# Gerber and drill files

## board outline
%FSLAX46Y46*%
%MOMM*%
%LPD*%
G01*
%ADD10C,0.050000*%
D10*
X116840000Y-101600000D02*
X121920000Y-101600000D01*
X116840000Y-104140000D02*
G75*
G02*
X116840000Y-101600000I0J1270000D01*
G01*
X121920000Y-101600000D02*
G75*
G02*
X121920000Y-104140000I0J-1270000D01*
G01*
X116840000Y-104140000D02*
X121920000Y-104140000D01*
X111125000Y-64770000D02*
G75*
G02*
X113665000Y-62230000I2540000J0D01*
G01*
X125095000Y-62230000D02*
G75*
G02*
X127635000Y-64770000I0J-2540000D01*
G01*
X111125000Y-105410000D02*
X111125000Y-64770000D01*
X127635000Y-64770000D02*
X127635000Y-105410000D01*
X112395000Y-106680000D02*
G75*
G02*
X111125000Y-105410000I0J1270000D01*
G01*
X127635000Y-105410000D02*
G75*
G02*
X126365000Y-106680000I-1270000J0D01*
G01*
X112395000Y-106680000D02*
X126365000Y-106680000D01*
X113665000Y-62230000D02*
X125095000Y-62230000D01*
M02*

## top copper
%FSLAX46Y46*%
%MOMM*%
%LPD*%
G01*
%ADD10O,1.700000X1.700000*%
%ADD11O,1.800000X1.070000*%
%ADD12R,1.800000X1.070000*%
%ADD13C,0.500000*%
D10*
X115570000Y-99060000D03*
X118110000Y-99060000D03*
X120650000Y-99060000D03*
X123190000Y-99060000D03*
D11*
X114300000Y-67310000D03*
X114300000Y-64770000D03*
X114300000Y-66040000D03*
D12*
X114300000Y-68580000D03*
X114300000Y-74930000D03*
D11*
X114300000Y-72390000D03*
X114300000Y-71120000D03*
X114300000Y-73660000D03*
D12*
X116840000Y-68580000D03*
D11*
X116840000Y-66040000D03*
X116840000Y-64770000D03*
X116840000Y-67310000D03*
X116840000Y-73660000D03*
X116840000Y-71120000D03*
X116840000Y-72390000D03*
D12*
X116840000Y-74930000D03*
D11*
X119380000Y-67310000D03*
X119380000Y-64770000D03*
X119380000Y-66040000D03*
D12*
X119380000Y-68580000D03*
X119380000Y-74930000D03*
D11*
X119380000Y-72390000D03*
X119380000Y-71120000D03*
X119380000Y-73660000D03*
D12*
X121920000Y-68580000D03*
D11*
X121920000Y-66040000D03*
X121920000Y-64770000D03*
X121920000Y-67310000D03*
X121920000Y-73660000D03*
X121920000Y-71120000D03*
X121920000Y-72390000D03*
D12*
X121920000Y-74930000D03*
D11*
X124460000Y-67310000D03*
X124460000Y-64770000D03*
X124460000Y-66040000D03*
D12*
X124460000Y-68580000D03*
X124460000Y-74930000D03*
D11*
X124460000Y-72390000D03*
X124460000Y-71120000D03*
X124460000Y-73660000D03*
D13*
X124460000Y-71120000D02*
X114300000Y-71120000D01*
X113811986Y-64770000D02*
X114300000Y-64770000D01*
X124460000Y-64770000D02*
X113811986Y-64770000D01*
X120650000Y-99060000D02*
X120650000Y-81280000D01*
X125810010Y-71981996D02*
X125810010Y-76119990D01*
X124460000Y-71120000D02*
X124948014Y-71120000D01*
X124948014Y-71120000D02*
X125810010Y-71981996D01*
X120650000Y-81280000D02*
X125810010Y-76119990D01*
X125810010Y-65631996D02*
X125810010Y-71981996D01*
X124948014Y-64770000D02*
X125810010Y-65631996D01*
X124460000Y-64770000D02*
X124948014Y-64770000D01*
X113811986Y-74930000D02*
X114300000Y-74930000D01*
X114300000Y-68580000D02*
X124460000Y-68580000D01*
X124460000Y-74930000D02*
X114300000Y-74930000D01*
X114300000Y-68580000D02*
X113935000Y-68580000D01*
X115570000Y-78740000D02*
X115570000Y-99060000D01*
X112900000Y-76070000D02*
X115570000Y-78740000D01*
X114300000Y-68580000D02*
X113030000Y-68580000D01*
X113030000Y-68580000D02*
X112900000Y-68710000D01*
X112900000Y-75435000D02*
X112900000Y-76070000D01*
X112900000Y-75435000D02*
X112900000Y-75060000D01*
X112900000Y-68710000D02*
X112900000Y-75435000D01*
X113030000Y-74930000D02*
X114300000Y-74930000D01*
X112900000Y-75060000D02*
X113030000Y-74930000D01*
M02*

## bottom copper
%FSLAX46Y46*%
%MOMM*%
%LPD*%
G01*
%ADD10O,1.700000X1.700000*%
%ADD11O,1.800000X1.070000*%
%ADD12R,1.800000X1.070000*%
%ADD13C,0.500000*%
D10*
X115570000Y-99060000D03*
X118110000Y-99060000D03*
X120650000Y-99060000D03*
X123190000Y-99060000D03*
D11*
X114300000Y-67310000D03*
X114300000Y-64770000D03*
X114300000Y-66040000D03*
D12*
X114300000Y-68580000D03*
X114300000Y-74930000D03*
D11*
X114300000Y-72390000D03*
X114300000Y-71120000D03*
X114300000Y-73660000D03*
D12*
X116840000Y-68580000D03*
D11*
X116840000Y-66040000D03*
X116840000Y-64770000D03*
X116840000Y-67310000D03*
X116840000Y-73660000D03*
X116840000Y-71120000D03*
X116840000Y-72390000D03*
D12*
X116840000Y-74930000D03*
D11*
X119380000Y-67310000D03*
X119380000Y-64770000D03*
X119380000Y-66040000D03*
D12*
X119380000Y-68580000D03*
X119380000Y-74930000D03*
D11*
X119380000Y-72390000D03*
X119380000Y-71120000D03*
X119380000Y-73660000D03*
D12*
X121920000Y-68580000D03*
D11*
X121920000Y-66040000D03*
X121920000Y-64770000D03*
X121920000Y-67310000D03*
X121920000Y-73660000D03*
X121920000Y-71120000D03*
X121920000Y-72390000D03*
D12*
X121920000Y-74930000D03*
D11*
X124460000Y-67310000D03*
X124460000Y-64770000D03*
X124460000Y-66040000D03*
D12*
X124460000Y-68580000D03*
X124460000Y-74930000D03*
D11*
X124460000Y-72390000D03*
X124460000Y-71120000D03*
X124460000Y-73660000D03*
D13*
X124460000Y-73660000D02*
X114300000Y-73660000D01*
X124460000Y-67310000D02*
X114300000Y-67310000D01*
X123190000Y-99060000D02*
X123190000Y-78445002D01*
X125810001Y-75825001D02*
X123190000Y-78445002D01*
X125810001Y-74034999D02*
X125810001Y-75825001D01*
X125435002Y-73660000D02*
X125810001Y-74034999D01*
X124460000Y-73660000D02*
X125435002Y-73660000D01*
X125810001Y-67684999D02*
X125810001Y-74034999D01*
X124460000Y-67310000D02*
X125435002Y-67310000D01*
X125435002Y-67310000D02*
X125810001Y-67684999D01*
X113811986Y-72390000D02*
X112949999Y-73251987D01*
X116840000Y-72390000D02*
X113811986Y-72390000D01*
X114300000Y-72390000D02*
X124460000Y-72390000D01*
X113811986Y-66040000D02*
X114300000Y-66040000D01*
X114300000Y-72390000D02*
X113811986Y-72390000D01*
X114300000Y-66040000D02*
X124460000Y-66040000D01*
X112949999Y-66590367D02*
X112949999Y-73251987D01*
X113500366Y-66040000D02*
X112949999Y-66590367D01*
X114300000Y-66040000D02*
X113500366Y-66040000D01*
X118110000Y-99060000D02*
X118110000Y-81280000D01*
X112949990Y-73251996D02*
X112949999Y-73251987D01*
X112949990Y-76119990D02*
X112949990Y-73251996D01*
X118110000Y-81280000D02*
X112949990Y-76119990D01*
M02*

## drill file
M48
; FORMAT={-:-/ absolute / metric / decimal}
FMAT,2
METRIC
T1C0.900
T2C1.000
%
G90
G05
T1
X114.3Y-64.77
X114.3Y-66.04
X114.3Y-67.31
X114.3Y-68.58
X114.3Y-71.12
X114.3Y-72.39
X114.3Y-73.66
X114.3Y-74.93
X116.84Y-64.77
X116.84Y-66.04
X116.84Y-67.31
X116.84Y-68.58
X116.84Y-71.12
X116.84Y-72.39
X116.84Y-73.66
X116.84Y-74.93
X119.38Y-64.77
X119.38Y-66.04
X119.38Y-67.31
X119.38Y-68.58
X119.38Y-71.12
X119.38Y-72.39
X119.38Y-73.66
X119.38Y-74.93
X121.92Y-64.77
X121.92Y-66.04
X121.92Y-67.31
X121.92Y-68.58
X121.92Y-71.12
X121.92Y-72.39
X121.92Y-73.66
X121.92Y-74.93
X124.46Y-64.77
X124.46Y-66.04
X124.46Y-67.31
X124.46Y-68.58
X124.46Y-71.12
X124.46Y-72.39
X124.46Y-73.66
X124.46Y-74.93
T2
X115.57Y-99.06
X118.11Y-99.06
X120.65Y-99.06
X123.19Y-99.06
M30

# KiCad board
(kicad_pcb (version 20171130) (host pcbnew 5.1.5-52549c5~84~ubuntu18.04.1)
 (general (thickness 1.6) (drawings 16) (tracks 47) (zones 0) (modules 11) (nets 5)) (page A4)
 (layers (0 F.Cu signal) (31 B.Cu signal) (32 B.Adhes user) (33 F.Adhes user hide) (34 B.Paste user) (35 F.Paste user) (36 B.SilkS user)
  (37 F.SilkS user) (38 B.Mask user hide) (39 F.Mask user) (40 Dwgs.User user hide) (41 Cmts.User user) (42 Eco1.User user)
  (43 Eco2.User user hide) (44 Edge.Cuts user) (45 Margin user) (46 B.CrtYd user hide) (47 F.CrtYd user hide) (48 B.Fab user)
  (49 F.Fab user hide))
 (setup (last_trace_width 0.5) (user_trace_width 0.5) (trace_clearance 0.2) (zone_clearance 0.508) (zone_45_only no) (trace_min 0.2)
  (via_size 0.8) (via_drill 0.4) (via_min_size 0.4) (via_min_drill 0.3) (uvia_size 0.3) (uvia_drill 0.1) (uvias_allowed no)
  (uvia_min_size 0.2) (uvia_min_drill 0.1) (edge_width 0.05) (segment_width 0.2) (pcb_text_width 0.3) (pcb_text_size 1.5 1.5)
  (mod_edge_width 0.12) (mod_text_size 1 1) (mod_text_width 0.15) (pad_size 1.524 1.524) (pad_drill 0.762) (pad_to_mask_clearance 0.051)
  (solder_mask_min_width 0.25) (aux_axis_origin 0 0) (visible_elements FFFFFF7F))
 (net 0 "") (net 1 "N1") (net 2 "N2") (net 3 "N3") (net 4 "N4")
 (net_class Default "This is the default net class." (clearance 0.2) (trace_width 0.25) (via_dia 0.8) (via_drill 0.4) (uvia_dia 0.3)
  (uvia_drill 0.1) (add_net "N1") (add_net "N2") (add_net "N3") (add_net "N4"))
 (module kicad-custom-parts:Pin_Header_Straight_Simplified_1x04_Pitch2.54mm (layer F.Cu) (at 115.57 99.06 90)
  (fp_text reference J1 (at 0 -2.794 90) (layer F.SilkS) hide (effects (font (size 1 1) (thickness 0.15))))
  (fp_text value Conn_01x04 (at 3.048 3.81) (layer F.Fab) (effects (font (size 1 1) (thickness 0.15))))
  (pad 1 thru_hole oval (at 0 0 90) (size 1.7 1.7) (drill 1) (layers *.Cu *.Mask) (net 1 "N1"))
  (pad 2 thru_hole oval (at 0 2.54 90) (size 1.7 1.7) (drill 1) (layers *.Cu *.Mask) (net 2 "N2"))
  (pad 3 thru_hole oval (at 0 5.08 90) (size 1.7 1.7) (drill 1) (layers *.Cu *.Mask) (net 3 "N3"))
  (pad 4 thru_hole oval (at 0 7.62 90) (size 1.7 1.7) (drill 1) (layers *.Cu *.Mask) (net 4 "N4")))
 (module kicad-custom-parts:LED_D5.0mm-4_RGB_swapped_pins (layer F.Cu) (at 114.3 68.58 90)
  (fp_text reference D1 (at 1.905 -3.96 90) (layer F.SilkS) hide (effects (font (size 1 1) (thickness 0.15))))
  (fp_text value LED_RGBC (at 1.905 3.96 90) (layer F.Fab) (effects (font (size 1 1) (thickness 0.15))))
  (pad 4 thru_hole oval (at 1.27 0 90) (size 1.07 1.8) (drill 0.9) (layers *.Cu *.Mask) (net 4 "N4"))
  (pad 3 thru_hole oval (at 3.81 0 90) (size 1.07 1.8) (drill 0.9) (layers *.Cu *.Mask) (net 3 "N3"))
  (pad 2 thru_hole oval (at 2.54 0 90) (size 1.07 1.8) (drill 0.9) (layers *.Cu *.Mask) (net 2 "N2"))
  (pad 1 thru_hole rect (at 0 0 90) (size 1.07 1.8) (drill 0.9) (layers *.Cu *.Mask) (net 1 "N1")))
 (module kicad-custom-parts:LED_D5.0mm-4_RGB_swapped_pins (layer F.Cu) (at 114.3 74.93 90)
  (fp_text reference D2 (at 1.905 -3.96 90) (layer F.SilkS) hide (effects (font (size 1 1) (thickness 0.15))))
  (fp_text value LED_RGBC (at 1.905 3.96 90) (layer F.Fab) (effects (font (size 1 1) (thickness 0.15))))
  (pad 1 thru_hole rect (at 0 0 90) (size 1.07 1.8) (drill 0.9) (layers *.Cu *.Mask) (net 1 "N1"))
  (pad 2 thru_hole oval (at 2.54 0 90) (size 1.07 1.8) (drill 0.9) (layers *.Cu *.Mask) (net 2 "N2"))
  (pad 3 thru_hole oval (at 3.81 0 90) (size 1.07 1.8) (drill 0.9) (layers *.Cu *.Mask) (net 3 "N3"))
  (pad 4 thru_hole oval (at 1.27 0 90) (size 1.07 1.8) (drill 0.9) (layers *.Cu *.Mask) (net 4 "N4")))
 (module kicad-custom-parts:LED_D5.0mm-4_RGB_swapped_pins (layer F.Cu) (at 116.84 68.58 90)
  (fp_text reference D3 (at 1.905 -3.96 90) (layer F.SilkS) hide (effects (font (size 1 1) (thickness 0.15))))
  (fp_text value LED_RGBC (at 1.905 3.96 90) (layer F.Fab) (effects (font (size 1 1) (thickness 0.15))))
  (pad 1 thru_hole rect (at 0 0 90) (size 1.07 1.8) (drill 0.9) (layers *.Cu *.Mask) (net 1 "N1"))
  (pad 2 thru_hole oval (at 2.54 0 90) (size 1.07 1.8) (drill 0.9) (layers *.Cu *.Mask) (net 2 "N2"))
  (pad 3 thru_hole oval (at 3.81 0 90) (size 1.07 1.8) (drill 0.9) (layers *.Cu *.Mask) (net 3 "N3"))
  (pad 4 thru_hole oval (at 1.27 0 90) (size 1.07 1.8) (drill 0.9) (layers *.Cu *.Mask) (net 4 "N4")))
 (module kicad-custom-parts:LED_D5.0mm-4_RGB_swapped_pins (layer F.Cu) (at 116.84 74.93 90)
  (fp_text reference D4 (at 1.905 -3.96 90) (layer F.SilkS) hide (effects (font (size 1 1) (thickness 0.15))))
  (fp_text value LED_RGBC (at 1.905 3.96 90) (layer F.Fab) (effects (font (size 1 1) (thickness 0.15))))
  (pad 4 thru_hole oval (at 1.27 0 90) (size 1.07 1.8) (drill 0.9) (layers *.Cu *.Mask) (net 4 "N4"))
  (pad 3 thru_hole oval (at 3.81 0 90) (size 1.07 1.8) (drill 0.9) (layers *.Cu *.Mask) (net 3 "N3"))
  (pad 2 thru_hole oval (at 2.54 0 90) (size 1.07 1.8) (drill 0.9) (layers *.Cu *.Mask) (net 2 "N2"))
  (pad 1 thru_hole rect (at 0 0 90) (size 1.07 1.8) (drill 0.9) (layers *.Cu *.Mask) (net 1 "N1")))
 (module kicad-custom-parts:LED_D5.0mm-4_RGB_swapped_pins (layer F.Cu) (at 119.38 68.58 90)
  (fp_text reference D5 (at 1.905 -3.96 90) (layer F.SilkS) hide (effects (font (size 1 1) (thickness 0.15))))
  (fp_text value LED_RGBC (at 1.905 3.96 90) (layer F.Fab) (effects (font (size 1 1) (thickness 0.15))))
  (pad 4 thru_hole oval (at 1.27 0 90) (size 1.07 1.8) (drill 0.9) (layers *.Cu *.Mask) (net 4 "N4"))
  (pad 3 thru_hole oval (at 3.81 0 90) (size 1.07 1.8) (drill 0.9) (layers *.Cu *.Mask) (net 3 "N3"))
  (pad 2 thru_hole oval (at 2.54 0 90) (size 1.07 1.8) (drill 0.9) (layers *.Cu *.Mask) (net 2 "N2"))
  (pad 1 thru_hole rect (at 0 0 90) (size 1.07 1.8) (drill 0.9) (layers *.Cu *.Mask) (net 1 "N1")))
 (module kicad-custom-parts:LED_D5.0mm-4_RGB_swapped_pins (layer F.Cu) (at 119.38 74.93 90)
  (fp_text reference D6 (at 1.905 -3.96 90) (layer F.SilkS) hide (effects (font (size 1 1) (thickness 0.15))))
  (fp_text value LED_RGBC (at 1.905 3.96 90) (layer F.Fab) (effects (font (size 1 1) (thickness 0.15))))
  (pad 1 thru_hole rect (at 0 0 90) (size 1.07 1.8) (drill 0.9) (layers *.Cu *.Mask) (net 1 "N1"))
  (pad 2 thru_hole oval (at 2.54 0 90) (size 1.07 1.8) (drill 0.9) (layers *.Cu *.Mask) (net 2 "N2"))
  (pad 3 thru_hole oval (at 3.81 0 90) (size 1.07 1.8) (drill 0.9) (layers *.Cu *.Mask) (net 3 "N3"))
  (pad 4 thru_hole oval (at 1.27 0 90) (size 1.07 1.8) (drill 0.9) (layers *.Cu *.Mask) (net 4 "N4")))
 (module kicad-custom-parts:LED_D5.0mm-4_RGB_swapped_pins (layer F.Cu) (at 121.92 68.58 90)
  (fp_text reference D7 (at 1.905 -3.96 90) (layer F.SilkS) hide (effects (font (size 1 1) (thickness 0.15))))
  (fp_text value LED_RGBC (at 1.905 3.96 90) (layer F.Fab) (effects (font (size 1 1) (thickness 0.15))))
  (pad 1 thru_hole rect (at 0 0 90) (size 1.07 1.8) (drill 0.9) (layers *.Cu *.Mask) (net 1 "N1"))
  (pad 2 thru_hole oval (at 2.54 0 90) (size 1.07 1.8) (drill 0.9) (layers *.Cu *.Mask) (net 2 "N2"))
  (pad 3 thru_hole oval (at 3.81 0 90) (size 1.07 1.8) (drill 0.9) (layers *.Cu *.Mask) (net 3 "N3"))
  (pad 4 thru_hole oval (at 1.27 0 90) (size 1.07 1.8) (drill 0.9) (layers *.Cu *.Mask) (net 4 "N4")))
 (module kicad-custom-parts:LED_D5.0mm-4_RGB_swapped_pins (layer F.Cu) (at 121.92 74.93 90)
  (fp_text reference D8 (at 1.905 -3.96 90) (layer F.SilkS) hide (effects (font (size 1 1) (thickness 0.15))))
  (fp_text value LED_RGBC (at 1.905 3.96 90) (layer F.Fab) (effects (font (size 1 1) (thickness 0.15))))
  (pad 4 thru_hole oval (at 1.27 0 90) (size 1.07 1.8) (drill 0.9) (layers *.Cu *.Mask) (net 4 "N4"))
  (pad 3 thru_hole oval (at 3.81 0 90) (size 1.07 1.8) (drill 0.9) (layers *.Cu *.Mask) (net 3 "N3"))
  (pad 2 thru_hole oval (at 2.54 0 90) (size 1.07 1.8) (drill 0.9) (layers *.Cu *.Mask) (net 2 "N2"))
  (pad 1 thru_hole rect (at 0 0 90) (size 1.07 1.8) (drill 0.9) (layers *.Cu *.Mask) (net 1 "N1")))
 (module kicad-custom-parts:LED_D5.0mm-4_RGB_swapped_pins (layer F.Cu) (at 124.46 68.58 90)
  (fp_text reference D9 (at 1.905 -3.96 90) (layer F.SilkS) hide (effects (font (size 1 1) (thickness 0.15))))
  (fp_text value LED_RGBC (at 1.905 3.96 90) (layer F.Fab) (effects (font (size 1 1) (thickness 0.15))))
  (pad 4 thru_hole oval (at 1.27 0 90) (size 1.07 1.8) (drill 0.9) (layers *.Cu *.Mask) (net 4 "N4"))
  (pad 3 thru_hole oval (at 3.81 0 90) (size 1.07 1.8) (drill 0.9) (layers *.Cu *.Mask) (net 3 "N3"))
  (pad 2 thru_hole oval (at 2.54 0 90) (size 1.07 1.8) (drill 0.9) (layers *.Cu *.Mask) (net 2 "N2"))
  (pad 1 thru_hole rect (at 0 0 90) (size 1.07 1.8) (drill 0.9) (layers *.Cu *.Mask) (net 1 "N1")))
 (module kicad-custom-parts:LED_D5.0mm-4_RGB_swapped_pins (layer F.Cu) (at 124.46 74.93 90)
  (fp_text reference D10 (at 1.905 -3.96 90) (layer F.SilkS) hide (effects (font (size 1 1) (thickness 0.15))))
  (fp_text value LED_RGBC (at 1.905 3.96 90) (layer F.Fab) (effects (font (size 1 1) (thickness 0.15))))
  (pad 1 thru_hole rect (at 0 0 90) (size 1.07 1.8) (drill 0.9) (layers *.Cu *.Mask) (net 1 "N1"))
  (pad 2 thru_hole oval (at 2.54 0 90) (size 1.07 1.8) (drill 0.9) (layers *.Cu *.Mask) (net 2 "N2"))
  (pad 3 thru_hole oval (at 3.81 0 90) (size 1.07 1.8) (drill 0.9) (layers *.Cu *.Mask) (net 3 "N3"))
  (pad 4 thru_hole oval (at 1.27 0 90) (size 1.07 1.8) (drill 0.9) (layers *.Cu *.Mask) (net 4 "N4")))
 (gr_line (start 116.84 101.6) (end 121.92 101.6) (layer Edge.Cuts) (width 0.05))
 (gr_arc (start 116.84 102.87) (end 116.84 101.6) (angle -180) (layer Edge.Cuts) (width 0.05))
 (gr_arc (start 121.92 102.87) (end 121.92 104.14) (angle -180) (layer Edge.Cuts) (width 0.05))
 (gr_line (start 116.84 104.14) (end 121.92 104.14) (layer Edge.Cuts) (width 0.05))
 (gr_arc (start 113.665 64.77) (end 113.665 62.23) (angle -90) (layer Edge.Cuts) (width 0.05))
 (gr_arc (start 125.095 64.77) (end 127.635 64.77) (angle -90) (layer Edge.Cuts) (width 0.05))
 (gr_line (start 111.125 105.41) (end 111.125 64.77) (layer Edge.Cuts) (width 0.05))
 (gr_line (start 127.635 64.77) (end 127.635 105.41) (layer Edge.Cuts) (width 0.05))
 (gr_arc (start 112.395 105.41) (end 111.125 105.41) (angle -90) (layer Edge.Cuts) (width 0.05))
 (gr_arc (start 126.365 105.41) (end 126.365 106.68) (angle -90) (layer Edge.Cuts) (width 0.05))
 (gr_line (start 112.395 106.68) (end 126.365 106.68) (layer Edge.Cuts) (width 0.05))
 (gr_line (start 113.665 62.23) (end 125.095 62.23) (layer Edge.Cuts) (width 0.05))
 (segment (start 124.46 73.66) (end 114.3 73.66) (width 0.5) (layer B.Cu) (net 4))
 (segment (start 124.46 67.31) (end 114.3 67.31) (width 0.5) (layer B.Cu) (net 4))
 (segment (start 123.19 99.06) (end 123.19 78.445002) (width 0.5) (layer B.Cu) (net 4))
 (segment (start 125.810001 75.825001) (end 123.19 78.445002) (width 0.5) (layer B.Cu) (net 4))
 (segment (start 125.810001 74.034999) (end 125.810001 75.825001) (width 0.5) (layer B.Cu) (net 4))
 (segment (start 125.435002 73.66) (end 125.810001 74.034999) (width 0.5) (layer B.Cu) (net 4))
 (segment (start 124.46 73.66) (end 125.435002 73.66) (width 0.5) (layer B.Cu) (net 4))
 (segment (start 125.810001 67.684999) (end 125.810001 74.034999) (width 0.5) (layer B.Cu) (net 4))
 (segment (start 124.46 67.31) (end 125.435002 67.31) (width 0.5) (layer B.Cu) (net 4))
 (segment (start 125.435002 67.31) (end 125.810001 67.684999) (width 0.5) (layer B.Cu) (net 4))
 (segment (start 124.46 71.12) (end 114.3 71.12) (width 0.5) (layer F.Cu) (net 3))
 (segment (start 113.811986 64.77) (end 114.3 64.77) (width 0.5) (layer F.Cu) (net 3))
 (segment (start 124.46 64.77) (end 113.811986 64.77) (width 0.5) (layer F.Cu) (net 3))
 (segment (start 120.65 99.06) (end 120.65 81.28) (width 0.5) (layer F.Cu) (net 3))
 (segment (start 125.81001 71.981996) (end 125.81001 76.11999) (width 0.5) (layer F.Cu) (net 3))
 (segment (start 124.46 71.12) (end 124.948014 71.12) (width 0.5) (layer F.Cu) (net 3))
 (segment (start 124.948014 71.12) (end 125.81001 71.981996) (width 0.5) (layer F.Cu) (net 3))
 (segment (start 120.65 81.28) (end 125.81001 76.11999) (width 0.5) (layer F.Cu) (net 3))
 (segment (start 125.81001 65.631996) (end 125.81001 71.981996) (width 0.5) (layer F.Cu) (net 3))
 (segment (start 124.948014 64.77) (end 125.81001 65.631996) (width 0.5) (layer F.Cu) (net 3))
 (segment (start 124.46 64.77) (end 124.948014 64.77) (width 0.5) (layer F.Cu) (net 3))
 (segment (start 113.811986 72.39) (end 112.949999 73.251987) (width 0.5) (layer B.Cu) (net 2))
 (segment (start 116.84 72.39) (end 113.811986 72.39) (width 0.5) (layer B.Cu) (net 2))
 (segment (start 114.3 72.39) (end 124.46 72.39) (width 0.5) (layer B.Cu) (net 2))
 (segment (start 113.811986 66.04) (end 114.3 66.04) (width 0.5) (layer B.Cu) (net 2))
 (segment (start 114.3 72.39) (end 113.811986 72.39) (width 0.5) (layer B.Cu) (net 2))
 (segment (start 114.3 66.04) (end 124.46 66.04) (width 0.5) (layer B.Cu) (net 2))
 (segment (start 112.949999 66.590367) (end 112.949999 73.251987) (width 0.5) (layer B.Cu) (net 2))
 (segment (start 113.500366 66.04) (end 112.949999 66.590367) (width 0.5) (layer B.Cu) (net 2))
 (segment (start 114.3 66.04) (end 113.500366 66.04) (width 0.5) (layer B.Cu) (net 2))
 (segment (start 118.11 99.06) (end 118.11 81.28) (width 0.5) (layer B.Cu) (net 2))
 (segment (start 112.94999 73.251996) (end 112.949999 73.251987) (width 0.5) (layer B.Cu) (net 2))
 (segment (start 112.94999 76.11999) (end 112.94999 73.251996) (width 0.5) (layer B.Cu) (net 2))
 (segment (start 118.11 81.28) (end 112.94999 76.11999) (width 0.5) (layer B.Cu) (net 2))
 (segment (start 113.811986 74.93) (end 114.3 74.93) (width 0.5) (layer F.Cu) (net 1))
 (segment (start 114.3 68.58) (end 124.46 68.58) (width 0.5) (layer F.Cu) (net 1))
 (segment (start 124.46 74.93) (end 114.3 74.93) (width 0.5) (layer F.Cu) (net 1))
 (segment (start 114.3 68.58) (end 113.935 68.58) (width 0.5) (layer F.Cu) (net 1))
 (segment (start 115.57 78.74) (end 115.57 99.06) (width 0.5) (layer F.Cu) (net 1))
 (segment (start 112.9 76.07) (end 115.57 78.74) (width 0.5) (layer F.Cu) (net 1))
 (segment (start 114.3 68.58) (end 113.03 68.58) (width 0.5) (layer F.Cu) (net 1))
 (segment (start 113.03 68.58) (end 112.9 68.71) (width 0.5) (layer F.Cu) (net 1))
 (segment (start 112.9 75.435) (end 112.9 76.07) (width 0.5) (layer F.Cu) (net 1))
 (segment (start 112.9 75.435) (end 112.9 75.06) (width 0.5) (layer F.Cu) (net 1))
 (segment (start 112.9 68.71) (end 112.9 75.435) (width 0.5) (layer F.Cu) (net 1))
 (segment (start 113.03 74.93) (end 114.3 74.93) (width 0.5) (layer F.Cu) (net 1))
 (segment (start 112.9 75.06) (end 113.03 74.93) (width 0.5) (layer F.Cu) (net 1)))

